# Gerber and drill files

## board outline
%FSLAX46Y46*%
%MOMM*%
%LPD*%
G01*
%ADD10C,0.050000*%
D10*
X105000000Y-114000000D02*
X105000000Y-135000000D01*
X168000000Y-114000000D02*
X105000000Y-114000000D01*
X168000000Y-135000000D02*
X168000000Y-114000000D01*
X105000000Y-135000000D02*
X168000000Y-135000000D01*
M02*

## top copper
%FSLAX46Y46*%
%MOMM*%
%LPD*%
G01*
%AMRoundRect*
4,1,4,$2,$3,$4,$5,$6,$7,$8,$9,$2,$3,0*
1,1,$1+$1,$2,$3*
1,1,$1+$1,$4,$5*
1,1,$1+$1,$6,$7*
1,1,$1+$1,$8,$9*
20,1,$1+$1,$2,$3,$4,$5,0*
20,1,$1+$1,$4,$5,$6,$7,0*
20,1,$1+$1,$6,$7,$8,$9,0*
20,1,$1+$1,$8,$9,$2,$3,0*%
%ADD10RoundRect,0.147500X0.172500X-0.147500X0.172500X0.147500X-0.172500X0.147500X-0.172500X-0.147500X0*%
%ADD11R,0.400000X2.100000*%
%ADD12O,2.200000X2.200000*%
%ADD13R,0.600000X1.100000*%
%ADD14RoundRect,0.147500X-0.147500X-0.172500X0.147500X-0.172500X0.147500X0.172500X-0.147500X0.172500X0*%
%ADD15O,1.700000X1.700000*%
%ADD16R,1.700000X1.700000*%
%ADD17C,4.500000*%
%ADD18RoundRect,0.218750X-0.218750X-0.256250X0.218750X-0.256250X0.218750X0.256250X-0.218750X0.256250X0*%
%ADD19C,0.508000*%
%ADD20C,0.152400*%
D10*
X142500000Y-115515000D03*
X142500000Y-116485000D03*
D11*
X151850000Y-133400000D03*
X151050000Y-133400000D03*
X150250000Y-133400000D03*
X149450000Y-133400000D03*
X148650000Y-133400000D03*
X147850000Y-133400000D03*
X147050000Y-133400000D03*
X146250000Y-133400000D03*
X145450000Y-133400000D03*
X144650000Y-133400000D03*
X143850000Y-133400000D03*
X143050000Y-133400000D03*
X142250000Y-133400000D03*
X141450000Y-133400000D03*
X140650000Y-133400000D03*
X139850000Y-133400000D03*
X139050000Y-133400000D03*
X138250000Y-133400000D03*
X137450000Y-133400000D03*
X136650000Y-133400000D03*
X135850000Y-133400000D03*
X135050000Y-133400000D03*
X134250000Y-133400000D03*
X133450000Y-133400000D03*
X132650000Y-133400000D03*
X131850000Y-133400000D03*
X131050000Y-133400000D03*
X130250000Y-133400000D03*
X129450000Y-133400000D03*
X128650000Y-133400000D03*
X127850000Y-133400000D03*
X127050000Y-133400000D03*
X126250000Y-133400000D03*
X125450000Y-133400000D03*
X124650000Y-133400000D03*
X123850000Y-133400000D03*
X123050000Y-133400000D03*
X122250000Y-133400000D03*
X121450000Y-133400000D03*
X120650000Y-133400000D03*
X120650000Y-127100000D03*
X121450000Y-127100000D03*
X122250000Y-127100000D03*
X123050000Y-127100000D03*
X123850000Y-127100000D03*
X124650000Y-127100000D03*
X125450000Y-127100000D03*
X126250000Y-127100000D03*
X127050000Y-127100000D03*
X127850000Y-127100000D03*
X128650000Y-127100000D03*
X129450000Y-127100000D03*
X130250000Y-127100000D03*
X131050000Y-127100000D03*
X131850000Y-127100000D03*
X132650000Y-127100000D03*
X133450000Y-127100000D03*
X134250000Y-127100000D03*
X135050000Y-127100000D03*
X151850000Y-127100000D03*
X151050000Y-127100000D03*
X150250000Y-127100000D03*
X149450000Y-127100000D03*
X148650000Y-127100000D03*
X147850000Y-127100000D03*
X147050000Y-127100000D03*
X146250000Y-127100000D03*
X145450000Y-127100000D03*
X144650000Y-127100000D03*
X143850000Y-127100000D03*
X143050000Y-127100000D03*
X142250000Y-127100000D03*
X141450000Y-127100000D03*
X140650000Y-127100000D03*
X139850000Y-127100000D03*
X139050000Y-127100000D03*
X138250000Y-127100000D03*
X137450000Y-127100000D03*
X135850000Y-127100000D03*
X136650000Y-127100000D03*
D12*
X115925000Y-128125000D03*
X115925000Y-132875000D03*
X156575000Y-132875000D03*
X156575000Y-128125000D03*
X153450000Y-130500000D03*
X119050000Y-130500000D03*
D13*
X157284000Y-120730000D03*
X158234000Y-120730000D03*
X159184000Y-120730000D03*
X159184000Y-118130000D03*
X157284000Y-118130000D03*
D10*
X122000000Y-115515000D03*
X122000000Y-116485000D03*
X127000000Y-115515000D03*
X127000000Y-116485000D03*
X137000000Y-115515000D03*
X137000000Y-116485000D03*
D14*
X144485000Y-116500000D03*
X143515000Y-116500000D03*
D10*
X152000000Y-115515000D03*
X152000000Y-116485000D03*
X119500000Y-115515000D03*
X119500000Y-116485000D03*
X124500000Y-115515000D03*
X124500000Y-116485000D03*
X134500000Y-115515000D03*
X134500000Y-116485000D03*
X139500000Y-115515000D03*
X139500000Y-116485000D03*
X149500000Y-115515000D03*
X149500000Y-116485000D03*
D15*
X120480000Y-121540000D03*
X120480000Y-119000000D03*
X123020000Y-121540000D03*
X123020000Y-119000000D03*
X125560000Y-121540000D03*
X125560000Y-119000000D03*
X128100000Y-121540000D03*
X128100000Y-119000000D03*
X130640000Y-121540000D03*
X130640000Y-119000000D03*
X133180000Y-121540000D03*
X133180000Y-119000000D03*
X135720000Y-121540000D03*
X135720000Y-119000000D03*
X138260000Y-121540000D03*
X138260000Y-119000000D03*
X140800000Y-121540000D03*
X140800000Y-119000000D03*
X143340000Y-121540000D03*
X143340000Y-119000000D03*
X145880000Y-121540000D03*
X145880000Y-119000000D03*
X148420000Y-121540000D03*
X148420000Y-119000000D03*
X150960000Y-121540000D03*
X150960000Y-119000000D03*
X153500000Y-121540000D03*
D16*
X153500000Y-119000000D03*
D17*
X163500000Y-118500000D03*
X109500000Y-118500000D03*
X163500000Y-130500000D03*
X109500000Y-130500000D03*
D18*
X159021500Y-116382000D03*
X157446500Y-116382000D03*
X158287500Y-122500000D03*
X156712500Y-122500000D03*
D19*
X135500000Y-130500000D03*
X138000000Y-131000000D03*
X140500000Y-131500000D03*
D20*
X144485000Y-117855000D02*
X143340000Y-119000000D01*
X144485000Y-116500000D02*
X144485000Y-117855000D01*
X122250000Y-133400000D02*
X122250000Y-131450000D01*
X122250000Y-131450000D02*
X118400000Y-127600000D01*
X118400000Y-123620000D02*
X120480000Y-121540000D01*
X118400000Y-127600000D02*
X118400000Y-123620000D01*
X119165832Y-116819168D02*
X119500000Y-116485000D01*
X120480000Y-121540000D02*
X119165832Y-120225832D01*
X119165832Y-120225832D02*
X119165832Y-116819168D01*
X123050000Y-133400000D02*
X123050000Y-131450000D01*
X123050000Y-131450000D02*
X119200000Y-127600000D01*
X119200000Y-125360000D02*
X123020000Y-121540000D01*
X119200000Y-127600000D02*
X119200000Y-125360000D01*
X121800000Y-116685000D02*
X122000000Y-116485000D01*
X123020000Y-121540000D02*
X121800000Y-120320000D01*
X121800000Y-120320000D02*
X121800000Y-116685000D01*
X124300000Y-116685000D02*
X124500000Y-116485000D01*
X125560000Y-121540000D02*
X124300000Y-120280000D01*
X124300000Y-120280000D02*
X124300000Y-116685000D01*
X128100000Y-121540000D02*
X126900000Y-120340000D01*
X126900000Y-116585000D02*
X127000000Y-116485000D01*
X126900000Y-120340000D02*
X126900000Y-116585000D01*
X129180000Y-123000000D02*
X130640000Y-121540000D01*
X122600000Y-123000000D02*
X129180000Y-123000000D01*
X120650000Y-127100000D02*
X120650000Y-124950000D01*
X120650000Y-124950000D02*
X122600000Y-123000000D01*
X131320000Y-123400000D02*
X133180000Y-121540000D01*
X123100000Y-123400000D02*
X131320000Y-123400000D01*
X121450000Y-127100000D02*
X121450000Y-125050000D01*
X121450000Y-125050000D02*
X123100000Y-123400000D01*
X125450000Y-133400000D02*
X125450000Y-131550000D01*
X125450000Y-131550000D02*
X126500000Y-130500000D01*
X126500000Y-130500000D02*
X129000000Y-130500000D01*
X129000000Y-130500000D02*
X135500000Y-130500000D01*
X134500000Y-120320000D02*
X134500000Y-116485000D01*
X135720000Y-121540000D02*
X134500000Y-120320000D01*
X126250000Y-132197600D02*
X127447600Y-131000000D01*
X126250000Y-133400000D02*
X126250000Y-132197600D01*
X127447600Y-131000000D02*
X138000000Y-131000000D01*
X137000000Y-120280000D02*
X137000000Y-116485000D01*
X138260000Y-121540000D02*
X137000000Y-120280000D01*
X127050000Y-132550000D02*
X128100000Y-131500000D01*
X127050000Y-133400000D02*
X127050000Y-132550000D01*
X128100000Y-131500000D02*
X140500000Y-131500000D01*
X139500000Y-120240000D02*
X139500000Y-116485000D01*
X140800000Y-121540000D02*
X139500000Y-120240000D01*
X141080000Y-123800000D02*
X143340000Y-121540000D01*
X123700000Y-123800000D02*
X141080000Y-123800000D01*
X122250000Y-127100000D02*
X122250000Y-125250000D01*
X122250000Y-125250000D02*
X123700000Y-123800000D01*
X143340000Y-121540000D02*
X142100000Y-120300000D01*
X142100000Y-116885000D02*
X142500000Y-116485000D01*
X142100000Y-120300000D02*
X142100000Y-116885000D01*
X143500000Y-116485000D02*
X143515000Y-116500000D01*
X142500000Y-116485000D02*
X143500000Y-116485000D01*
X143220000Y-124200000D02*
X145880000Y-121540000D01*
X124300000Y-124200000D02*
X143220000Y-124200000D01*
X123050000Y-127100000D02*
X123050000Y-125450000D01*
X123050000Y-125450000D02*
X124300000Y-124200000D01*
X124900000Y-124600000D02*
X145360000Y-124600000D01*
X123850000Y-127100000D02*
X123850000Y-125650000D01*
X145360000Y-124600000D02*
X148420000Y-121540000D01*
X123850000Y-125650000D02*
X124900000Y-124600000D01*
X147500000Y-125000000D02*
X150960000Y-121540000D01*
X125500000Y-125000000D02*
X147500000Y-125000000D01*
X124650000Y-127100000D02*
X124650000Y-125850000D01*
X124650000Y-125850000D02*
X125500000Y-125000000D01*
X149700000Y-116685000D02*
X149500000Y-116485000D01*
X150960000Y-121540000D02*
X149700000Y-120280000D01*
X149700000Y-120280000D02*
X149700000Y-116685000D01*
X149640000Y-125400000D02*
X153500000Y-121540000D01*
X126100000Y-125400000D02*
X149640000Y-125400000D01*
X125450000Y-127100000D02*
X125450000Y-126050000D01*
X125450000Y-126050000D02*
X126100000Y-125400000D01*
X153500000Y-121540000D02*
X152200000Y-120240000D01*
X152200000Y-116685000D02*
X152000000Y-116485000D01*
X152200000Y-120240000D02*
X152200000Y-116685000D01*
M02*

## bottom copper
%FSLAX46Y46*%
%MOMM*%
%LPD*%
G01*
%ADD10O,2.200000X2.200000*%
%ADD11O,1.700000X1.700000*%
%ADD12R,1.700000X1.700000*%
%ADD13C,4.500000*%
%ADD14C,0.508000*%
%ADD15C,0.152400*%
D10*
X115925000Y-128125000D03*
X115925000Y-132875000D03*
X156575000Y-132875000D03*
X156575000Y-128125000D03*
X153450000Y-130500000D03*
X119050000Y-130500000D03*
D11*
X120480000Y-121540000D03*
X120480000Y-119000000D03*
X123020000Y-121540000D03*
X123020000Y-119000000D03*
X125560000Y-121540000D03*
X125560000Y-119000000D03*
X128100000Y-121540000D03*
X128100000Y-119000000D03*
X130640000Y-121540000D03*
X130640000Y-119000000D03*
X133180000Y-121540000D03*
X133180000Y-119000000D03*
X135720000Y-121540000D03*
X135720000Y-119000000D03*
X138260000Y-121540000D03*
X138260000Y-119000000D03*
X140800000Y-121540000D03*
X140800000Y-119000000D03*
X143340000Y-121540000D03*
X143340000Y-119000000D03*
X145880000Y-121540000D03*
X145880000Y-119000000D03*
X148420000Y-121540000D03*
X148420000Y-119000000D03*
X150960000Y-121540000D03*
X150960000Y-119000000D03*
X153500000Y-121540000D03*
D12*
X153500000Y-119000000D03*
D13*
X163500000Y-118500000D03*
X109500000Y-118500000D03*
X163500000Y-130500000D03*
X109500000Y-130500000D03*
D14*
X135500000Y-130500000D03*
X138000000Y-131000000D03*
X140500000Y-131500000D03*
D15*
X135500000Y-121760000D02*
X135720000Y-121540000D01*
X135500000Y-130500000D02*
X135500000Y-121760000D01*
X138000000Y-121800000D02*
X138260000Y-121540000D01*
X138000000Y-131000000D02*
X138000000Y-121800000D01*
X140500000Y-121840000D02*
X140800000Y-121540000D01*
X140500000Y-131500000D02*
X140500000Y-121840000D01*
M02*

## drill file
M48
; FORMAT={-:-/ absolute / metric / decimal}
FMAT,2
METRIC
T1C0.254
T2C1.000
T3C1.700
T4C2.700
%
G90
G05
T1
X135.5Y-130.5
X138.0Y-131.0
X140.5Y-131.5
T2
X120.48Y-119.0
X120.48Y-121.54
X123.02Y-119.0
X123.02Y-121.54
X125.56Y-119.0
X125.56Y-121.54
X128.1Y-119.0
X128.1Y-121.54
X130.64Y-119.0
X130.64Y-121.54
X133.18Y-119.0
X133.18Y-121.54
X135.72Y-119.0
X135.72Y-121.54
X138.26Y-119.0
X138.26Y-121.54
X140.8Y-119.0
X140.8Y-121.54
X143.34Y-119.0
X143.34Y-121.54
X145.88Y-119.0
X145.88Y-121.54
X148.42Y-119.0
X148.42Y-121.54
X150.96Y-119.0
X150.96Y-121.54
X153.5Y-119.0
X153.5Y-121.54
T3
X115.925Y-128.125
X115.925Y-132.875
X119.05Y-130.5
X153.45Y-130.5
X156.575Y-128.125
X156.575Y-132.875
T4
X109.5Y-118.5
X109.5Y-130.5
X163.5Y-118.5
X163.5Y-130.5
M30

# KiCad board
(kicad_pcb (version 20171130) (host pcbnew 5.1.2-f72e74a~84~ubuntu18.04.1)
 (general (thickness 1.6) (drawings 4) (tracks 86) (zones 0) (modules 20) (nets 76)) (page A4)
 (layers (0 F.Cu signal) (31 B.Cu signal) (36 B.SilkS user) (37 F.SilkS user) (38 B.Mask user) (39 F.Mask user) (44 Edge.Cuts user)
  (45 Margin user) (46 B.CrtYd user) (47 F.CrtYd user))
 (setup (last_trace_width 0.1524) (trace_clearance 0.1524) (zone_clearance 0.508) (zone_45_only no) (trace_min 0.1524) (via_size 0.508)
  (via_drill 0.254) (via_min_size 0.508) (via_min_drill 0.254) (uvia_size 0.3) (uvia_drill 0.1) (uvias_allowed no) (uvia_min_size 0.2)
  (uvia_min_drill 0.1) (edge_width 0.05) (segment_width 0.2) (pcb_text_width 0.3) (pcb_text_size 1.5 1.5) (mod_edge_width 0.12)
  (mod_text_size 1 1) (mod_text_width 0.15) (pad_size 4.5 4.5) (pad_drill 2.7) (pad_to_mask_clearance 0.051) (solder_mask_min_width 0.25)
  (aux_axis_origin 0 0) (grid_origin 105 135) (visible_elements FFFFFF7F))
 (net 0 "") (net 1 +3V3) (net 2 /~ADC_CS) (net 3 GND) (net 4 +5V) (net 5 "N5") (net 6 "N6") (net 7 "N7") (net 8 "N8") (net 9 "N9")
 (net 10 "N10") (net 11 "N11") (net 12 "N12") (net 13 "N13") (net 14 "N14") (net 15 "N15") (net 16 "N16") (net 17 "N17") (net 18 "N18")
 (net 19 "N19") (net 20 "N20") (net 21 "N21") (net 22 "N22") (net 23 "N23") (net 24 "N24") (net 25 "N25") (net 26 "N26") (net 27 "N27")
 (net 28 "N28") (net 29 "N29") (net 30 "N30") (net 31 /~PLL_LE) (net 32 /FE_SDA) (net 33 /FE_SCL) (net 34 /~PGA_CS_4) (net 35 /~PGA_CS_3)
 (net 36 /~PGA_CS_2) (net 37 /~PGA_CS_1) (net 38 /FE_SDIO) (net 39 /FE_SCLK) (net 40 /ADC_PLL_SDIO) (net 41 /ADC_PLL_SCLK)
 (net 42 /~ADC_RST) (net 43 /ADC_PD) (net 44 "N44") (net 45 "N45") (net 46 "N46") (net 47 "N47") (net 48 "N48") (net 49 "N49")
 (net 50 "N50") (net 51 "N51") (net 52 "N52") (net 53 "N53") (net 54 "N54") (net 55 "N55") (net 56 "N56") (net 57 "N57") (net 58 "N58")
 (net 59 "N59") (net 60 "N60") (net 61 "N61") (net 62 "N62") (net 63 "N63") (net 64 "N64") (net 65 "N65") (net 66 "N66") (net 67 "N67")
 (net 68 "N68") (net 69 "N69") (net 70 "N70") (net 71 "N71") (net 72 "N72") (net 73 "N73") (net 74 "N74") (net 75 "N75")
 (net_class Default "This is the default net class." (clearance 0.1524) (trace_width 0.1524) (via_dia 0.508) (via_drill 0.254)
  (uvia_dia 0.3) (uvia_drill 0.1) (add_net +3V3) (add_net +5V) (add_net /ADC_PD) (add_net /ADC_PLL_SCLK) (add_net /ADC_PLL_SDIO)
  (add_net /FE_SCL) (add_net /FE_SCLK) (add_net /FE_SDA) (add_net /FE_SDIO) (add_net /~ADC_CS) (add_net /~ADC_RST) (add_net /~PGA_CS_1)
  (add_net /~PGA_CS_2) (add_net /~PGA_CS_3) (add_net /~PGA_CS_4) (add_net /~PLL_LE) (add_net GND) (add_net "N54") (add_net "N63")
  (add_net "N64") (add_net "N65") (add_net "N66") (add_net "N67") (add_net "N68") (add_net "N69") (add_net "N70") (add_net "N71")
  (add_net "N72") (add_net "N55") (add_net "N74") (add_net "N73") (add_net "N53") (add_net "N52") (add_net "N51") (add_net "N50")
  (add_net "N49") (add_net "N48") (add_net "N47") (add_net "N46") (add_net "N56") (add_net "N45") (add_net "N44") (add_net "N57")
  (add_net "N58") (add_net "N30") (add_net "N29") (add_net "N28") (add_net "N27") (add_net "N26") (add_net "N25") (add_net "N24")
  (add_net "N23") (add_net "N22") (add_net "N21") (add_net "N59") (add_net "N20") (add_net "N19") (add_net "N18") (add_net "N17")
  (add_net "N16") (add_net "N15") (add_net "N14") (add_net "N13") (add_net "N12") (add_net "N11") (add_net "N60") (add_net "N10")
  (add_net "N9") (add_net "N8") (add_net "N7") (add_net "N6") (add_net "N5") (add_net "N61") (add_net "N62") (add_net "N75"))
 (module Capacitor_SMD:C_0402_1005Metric (layer F.Cu) (at 142.5 116 90)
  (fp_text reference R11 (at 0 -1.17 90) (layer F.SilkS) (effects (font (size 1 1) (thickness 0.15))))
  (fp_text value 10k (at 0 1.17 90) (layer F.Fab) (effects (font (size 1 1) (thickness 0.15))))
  (pad 2 smd roundrect (at 0.485 0 90) (size 0.59 0.64) (layers F.Cu F.Paste F.Mask) (roundrect_rratio 0.25) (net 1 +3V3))
  (pad 1 smd roundrect (at -0.485 0 90) (size 0.59 0.64) (layers F.Cu F.Paste F.Mask) (roundrect_rratio 0.25) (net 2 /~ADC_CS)))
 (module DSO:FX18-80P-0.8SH (layer F.Cu) (at 136.25 130.5 180)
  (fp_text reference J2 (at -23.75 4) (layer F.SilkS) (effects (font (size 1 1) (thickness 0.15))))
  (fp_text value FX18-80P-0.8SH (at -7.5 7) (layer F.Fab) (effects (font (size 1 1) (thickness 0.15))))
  (pad 80 smd rect (at -15.6 -2.9 180) (size 0.4 2.1) (layers F.Cu F.Paste F.Mask) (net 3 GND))
  (pad 79 smd rect (at -14.8 -2.9 180) (size 0.4 2.1) (layers F.Cu F.Paste F.Mask) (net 3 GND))
  (pad 78 smd rect (at -14 -2.9 180) (size 0.4 2.1) (layers F.Cu F.Paste F.Mask) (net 3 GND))
  (pad 77 smd rect (at -13.2 -2.9 180) (size 0.4 2.1) (layers F.Cu F.Paste F.Mask) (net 3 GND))
  (pad 76 smd rect (at -12.4 -2.9 180) (size 0.4 2.1) (layers F.Cu F.Paste F.Mask) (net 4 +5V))
  (pad 75 smd rect (at -11.6 -2.9 180) (size 0.4 2.1) (layers F.Cu F.Paste F.Mask) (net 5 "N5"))
  (pad 74 smd rect (at -10.8 -2.9 180) (size 0.4 2.1) (layers F.Cu F.Paste F.Mask) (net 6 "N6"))
  (pad 73 smd rect (at -10 -2.9 180) (size 0.4 2.1) (layers F.Cu F.Paste F.Mask) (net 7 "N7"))
  (pad 72 smd rect (at -9.2 -2.9 180) (size 0.4 2.1) (layers F.Cu F.Paste F.Mask) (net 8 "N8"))
  (pad 71 smd rect (at -8.4 -2.9 180) (size 0.4 2.1) (layers F.Cu F.Paste F.Mask) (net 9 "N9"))
  (pad 70 smd rect (at -7.6 -2.9 180) (size 0.4 2.1) (layers F.Cu F.Paste F.Mask) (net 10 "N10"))
  (pad 69 smd rect (at -6.8 -2.9 180) (size 0.4 2.1) (layers F.Cu F.Paste F.Mask) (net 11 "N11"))
  (pad 68 smd rect (at -6 -2.9 180) (size 0.4 2.1) (layers F.Cu F.Paste F.Mask) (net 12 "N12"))
  (pad 67 smd rect (at -5.2 -2.9 180) (size 0.4 2.1) (layers F.Cu F.Paste F.Mask) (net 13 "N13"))
  (pad 66 smd rect (at -4.4 -2.9 180) (size 0.4 2.1) (layers F.Cu F.Paste F.Mask) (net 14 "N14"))
  (pad 65 smd rect (at -3.6 -2.9 180) (size 0.4 2.1) (layers F.Cu F.Paste F.Mask) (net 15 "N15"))
  (pad 64 smd rect (at -2.8 -2.9 180) (size 0.4 2.1) (layers F.Cu F.Paste F.Mask) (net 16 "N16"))
  (pad 63 smd rect (at -2 -2.9 180) (size 0.4 2.1) (layers F.Cu F.Paste F.Mask) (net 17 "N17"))
  (pad 62 smd rect (at -1.2 -2.9 180) (size 0.4 2.1) (layers F.Cu F.Paste F.Mask) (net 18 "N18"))
  (pad 61 smd rect (at -0.4 -2.9 180) (size 0.4 2.1) (layers F.Cu F.Paste F.Mask) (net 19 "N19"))
  (pad 60 smd rect (at 0.4 -2.9 180) (size 0.4 2.1) (layers F.Cu F.Paste F.Mask) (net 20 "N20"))
  (pad 59 smd rect (at 1.2 -2.9 180) (size 0.4 2.1) (layers F.Cu F.Paste F.Mask) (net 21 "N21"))
  (pad 58 smd rect (at 2 -2.9 180) (size 0.4 2.1) (layers F.Cu F.Paste F.Mask) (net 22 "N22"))
  (pad 57 smd rect (at 2.8 -2.9 180) (size 0.4 2.1) (layers F.Cu F.Paste F.Mask) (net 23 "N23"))
  (pad 56 smd rect (at 3.6 -2.9 180) (size 0.4 2.1) (layers F.Cu F.Paste F.Mask) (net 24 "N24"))
  (pad 55 smd rect (at 4.4 -2.9 180) (size 0.4 2.1) (layers F.Cu F.Paste F.Mask) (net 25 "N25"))
  (pad 54 smd rect (at 5.2 -2.9 180) (size 0.4 2.1) (layers F.Cu F.Paste F.Mask) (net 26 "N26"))
  (pad 53 smd rect (at 6 -2.9 180) (size 0.4 2.1) (layers F.Cu F.Paste F.Mask) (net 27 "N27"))
  (pad 52 smd rect (at 6.8 -2.9 180) (size 0.4 2.1) (layers F.Cu F.Paste F.Mask) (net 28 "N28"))
  (pad 51 smd rect (at 7.6 -2.9 180) (size 0.4 2.1) (layers F.Cu F.Paste F.Mask) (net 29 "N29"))
  (pad 50 smd rect (at 8.4 -2.9 180) (size 0.4 2.1) (layers F.Cu F.Paste F.Mask) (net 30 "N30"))
  (pad 49 smd rect (at 9.2 -2.9 180) (size 0.4 2.1) (layers F.Cu F.Paste F.Mask) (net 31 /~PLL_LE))
  (pad 48 smd rect (at 10 -2.9 180) (size 0.4 2.1) (layers F.Cu F.Paste F.Mask) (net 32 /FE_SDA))
  (pad 47 smd rect (at 10.8 -2.9 180) (size 0.4 2.1) (layers F.Cu F.Paste F.Mask) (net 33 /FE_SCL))
  (pad 46 smd rect (at 11.6 -2.9 180) (size 0.4 2.1) (layers F.Cu F.Paste F.Mask) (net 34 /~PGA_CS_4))
  (pad 45 smd rect (at 12.4 -2.9 180) (size 0.4 2.1) (layers F.Cu F.Paste F.Mask) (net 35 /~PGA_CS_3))
  (pad 44 smd rect (at 13.2 -2.9 180) (size 0.4 2.1) (layers F.Cu F.Paste F.Mask) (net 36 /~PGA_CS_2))
  (pad 43 smd rect (at 14 -2.9 180) (size 0.4 2.1) (layers F.Cu F.Paste F.Mask) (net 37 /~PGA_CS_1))
  (pad 42 smd rect (at 14.8 -2.9 180) (size 0.4 2.1) (layers F.Cu F.Paste F.Mask) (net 3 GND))
  (pad 41 smd rect (at 15.6 -2.9 180) (size 0.4 2.1) (layers F.Cu F.Paste F.Mask) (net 3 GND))
  (pad 40 smd rect (at 15.6 3.4 180) (size 0.4 2.1) (layers F.Cu F.Paste F.Mask) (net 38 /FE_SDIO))
  (pad 39 smd rect (at 14.8 3.4 180) (size 0.4 2.1) (layers F.Cu F.Paste F.Mask) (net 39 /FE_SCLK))
  (pad 38 smd rect (at 14 3.4 180) (size 0.4 2.1) (layers F.Cu F.Paste F.Mask) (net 2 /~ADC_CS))
  (pad 37 smd rect (at 13.2 3.4 180) (size 0.4 2.1) (layers F.Cu F.Paste F.Mask) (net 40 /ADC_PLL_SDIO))
  (pad 36 smd rect (at 12.4 3.4 180) (size 0.4 2.1) (layers F.Cu F.Paste F.Mask) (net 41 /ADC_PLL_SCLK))
  (pad 35 smd rect (at 11.6 3.4 180) (size 0.4 2.1) (layers F.Cu F.Paste F.Mask) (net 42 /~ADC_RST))
  (pad 34 smd rect (at 10.8 3.4 180) (size 0.4 2.1) (layers F.Cu F.Paste F.Mask) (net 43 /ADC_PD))
  (pad 33 smd rect (at 10 3.4 180) (size 0.4 2.1) (layers F.Cu F.Paste F.Mask) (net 3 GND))
  (pad 32 smd rect (at 9.2 3.4 180) (size 0.4 2.1) (layers F.Cu F.Paste F.Mask) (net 3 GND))
  (pad 31 smd rect (at 8.4 3.4 180) (size 0.4 2.1) (layers F.Cu F.Paste F.Mask) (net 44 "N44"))
  (pad 30 smd rect (at 7.6 3.4 180) (size 0.4 2.1) (layers F.Cu F.Paste F.Mask) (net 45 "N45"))
  (pad 29 smd rect (at 6.8 3.4 180) (size 0.4 2.1) (layers F.Cu F.Paste F.Mask) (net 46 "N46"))
  (pad 28 smd rect (at 6 3.4 180) (size 0.4 2.1) (layers F.Cu F.Paste F.Mask) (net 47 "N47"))
  (pad 27 smd rect (at 5.2 3.4 180) (size 0.4 2.1) (layers F.Cu F.Paste F.Mask) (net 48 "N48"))
  (pad 26 smd rect (at 4.4 3.4 180) (size 0.4 2.1) (layers F.Cu F.Paste F.Mask) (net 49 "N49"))
  (pad 25 smd rect (at 3.6 3.4 180) (size 0.4 2.1) (layers F.Cu F.Paste F.Mask) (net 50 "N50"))
  (pad 24 smd rect (at 2.8 3.4 180) (size 0.4 2.1) (layers F.Cu F.Paste F.Mask) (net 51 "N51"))
  (pad 23 smd rect (at 2 3.4 180) (size 0.4 2.1) (layers F.Cu F.Paste F.Mask) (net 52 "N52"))
  (pad 22 smd rect (at 1.2 3.4 180) (size 0.4 2.1) (layers F.Cu F.Paste F.Mask) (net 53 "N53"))
  (pad 1 smd rect (at -15.6 3.4 180) (size 0.4 2.1) (layers F.Cu F.Paste F.Mask) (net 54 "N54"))
  (pad 2 smd rect (at -14.8 3.4 180) (size 0.4 2.1) (layers F.Cu F.Paste F.Mask) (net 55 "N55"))
  (pad 3 smd rect (at -14 3.4 180) (size 0.4 2.1) (layers F.Cu F.Paste F.Mask) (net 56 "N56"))
  (pad 4 smd rect (at -13.2 3.4 180) (size 0.4 2.1) (layers F.Cu F.Paste F.Mask) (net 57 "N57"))
  (pad 5 smd rect (at -12.4 3.4 180) (size 0.4 2.1) (layers F.Cu F.Paste F.Mask) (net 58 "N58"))
  (pad 6 smd rect (at -11.6 3.4 180) (size 0.4 2.1) (layers F.Cu F.Paste F.Mask) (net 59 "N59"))
  (pad 7 smd rect (at -10.8 3.4 180) (size 0.4 2.1) (layers F.Cu F.Paste F.Mask) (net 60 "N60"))
  (pad 8 smd rect (at -10 3.4 180) (size 0.4 2.1) (layers F.Cu F.Paste F.Mask) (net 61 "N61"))
  (pad 9 smd rect (at -9.2 3.4 180) (size 0.4 2.1) (layers F.Cu F.Paste F.Mask) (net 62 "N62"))
  (pad 10 smd rect (at -8.4 3.4 180) (size 0.4 2.1) (layers F.Cu F.Paste F.Mask) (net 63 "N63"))
  (pad 11 smd rect (at -7.6 3.4 180) (size 0.4 2.1) (layers F.Cu F.Paste F.Mask) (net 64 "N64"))
  (pad 12 smd rect (at -6.8 3.4 180) (size 0.4 2.1) (layers F.Cu F.Paste F.Mask) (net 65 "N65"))
  (pad 13 smd rect (at -6 3.4 180) (size 0.4 2.1) (layers F.Cu F.Paste F.Mask) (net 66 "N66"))
  (pad 14 smd rect (at -5.2 3.4 180) (size 0.4 2.1) (layers F.Cu F.Paste F.Mask) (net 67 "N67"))
  (pad 15 smd rect (at -4.4 3.4 180) (size 0.4 2.1) (layers F.Cu F.Paste F.Mask) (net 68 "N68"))
  (pad 16 smd rect (at -3.6 3.4 180) (size 0.4 2.1) (layers F.Cu F.Paste F.Mask) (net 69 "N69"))
  (pad 17 smd rect (at -2.8 3.4 180) (size 0.4 2.1) (layers F.Cu F.Paste F.Mask) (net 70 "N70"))
  (pad 18 smd rect (at -2 3.4 180) (size 0.4 2.1) (layers F.Cu F.Paste F.Mask) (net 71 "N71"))
  (pad 19 smd rect (at -1.2 3.4 180) (size 0.4 2.1) (layers F.Cu F.Paste F.Mask) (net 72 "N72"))
  (pad 21 smd rect (at 0.4 3.4 180) (size 0.4 2.1) (layers F.Cu F.Paste F.Mask) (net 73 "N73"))
  (pad 20 smd rect (at -0.4 3.4 180) (size 0.4 2.1) (layers F.Cu F.Paste F.Mask) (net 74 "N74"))
  (pad SHLD thru_hole oval (at 20.325 2.375 180) (size 2.2 2.2) (drill 1.7) (layers *.Cu *.Mask) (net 3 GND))
  (pad SHLD thru_hole oval (at 20.325 -2.375 180) (size 2.2 2.2) (drill 1.7) (layers *.Cu *.Mask) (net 3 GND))
  (pad SHLD thru_hole oval (at -20.325 -2.375 180) (size 2.2 2.2) (drill 1.7) (layers *.Cu *.Mask) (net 3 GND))
  (pad SHLD thru_hole oval (at -20.325 2.375 180) (size 2.2 2.2) (drill 1.7) (layers *.Cu *.Mask) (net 3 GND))
  (pad SHLD thru_hole oval (at -17.2 0 180) (size 2.2 2.2) (drill 1.7) (layers *.Cu *.Mask) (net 3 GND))
  (pad SHLD thru_hole oval (at 17.2 0 180) (size 2.2 2.2) (drill 1.7) (layers *.Cu *.Mask) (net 3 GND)))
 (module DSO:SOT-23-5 (layer F.Cu) (at 158.234 119.43 90) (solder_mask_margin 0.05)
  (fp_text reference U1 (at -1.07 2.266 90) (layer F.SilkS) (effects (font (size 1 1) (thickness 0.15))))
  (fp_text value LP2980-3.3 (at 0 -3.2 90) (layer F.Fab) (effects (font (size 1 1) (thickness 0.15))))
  (pad 1 smd rect (at -1.3 -0.95 90) (size 1.1 0.6) (layers F.Cu F.Paste F.Mask) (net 4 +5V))
  (pad 2 smd rect (at -1.3 0 90) (size 1.1 0.6) (layers F.Cu F.Paste F.Mask) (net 3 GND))
  (pad 3 smd rect (at -1.3 0.95 90) (size 1.1 0.6) (layers F.Cu F.Paste F.Mask) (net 4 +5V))
  (pad 4 smd rect (at 1.3 0.95 90) (size 1.1 0.6) (layers F.Cu F.Paste F.Mask) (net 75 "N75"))
  (pad 5 smd rect (at 1.3 -0.95 90) (size 1.1 0.6) (layers F.Cu F.Paste F.Mask) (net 1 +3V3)))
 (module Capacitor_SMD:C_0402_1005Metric (layer F.Cu) (at 122 116 90)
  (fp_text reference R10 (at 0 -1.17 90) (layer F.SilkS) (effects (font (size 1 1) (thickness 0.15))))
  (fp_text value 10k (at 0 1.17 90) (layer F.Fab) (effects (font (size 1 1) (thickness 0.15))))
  (pad 2 smd roundrect (at 0.485 0 90) (size 0.59 0.64) (layers F.Cu F.Paste F.Mask) (roundrect_rratio 0.25) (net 1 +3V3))
  (pad 1 smd roundrect (at -0.485 0 90) (size 0.59 0.64) (layers F.Cu F.Paste F.Mask) (roundrect_rratio 0.25) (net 36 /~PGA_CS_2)))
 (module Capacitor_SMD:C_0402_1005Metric (layer F.Cu) (at 127 116 90)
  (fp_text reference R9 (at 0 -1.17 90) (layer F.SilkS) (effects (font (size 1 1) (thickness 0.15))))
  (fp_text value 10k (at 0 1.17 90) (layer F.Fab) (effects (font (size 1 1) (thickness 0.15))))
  (pad 2 smd roundrect (at 0.485 0 90) (size 0.59 0.64) (layers F.Cu F.Paste F.Mask) (roundrect_rratio 0.25) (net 1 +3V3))
  (pad 1 smd roundrect (at -0.485 0 90) (size 0.59 0.64) (layers F.Cu F.Paste F.Mask) (roundrect_rratio 0.25) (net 34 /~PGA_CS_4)))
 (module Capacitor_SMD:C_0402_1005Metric (layer F.Cu) (at 137 116 90)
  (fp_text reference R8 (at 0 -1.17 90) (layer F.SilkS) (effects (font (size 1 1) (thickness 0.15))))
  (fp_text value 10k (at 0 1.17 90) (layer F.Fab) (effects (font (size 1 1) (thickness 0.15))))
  (pad 2 smd roundrect (at 0.485 0 90) (size 0.59 0.64) (layers F.Cu F.Paste F.Mask) (roundrect_rratio 0.25) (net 1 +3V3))
  (pad 1 smd roundrect (at -0.485 0 90) (size 0.59 0.64) (layers F.Cu F.Paste F.Mask) (roundrect_rratio 0.25) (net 32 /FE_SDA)))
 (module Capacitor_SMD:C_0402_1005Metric (layer F.Cu) (at 144 116.5)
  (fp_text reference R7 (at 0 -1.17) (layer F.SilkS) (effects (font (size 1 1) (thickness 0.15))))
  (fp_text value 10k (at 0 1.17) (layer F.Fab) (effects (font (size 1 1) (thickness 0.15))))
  (pad 2 smd roundrect (at 0.485 0) (size 0.59 0.64) (layers F.Cu F.Paste F.Mask) (roundrect_rratio 0.25) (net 3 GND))
  (pad 1 smd roundrect (at -0.485 0) (size 0.59 0.64) (layers F.Cu F.Paste F.Mask) (roundrect_rratio 0.25) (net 2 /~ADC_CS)))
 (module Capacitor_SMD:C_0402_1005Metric (layer F.Cu) (at 152 116 90)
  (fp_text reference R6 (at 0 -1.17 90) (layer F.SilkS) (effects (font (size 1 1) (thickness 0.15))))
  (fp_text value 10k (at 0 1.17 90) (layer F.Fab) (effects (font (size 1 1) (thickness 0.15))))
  (pad 2 smd roundrect (at 0.485 0 90) (size 0.59 0.64) (layers F.Cu F.Paste F.Mask) (roundrect_rratio 0.25) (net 1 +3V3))
  (pad 1 smd roundrect (at -0.485 0 90) (size 0.59 0.64) (layers F.Cu F.Paste F.Mask) (roundrect_rratio 0.25) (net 43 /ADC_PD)))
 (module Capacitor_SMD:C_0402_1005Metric (layer F.Cu) (at 119.5 116 90)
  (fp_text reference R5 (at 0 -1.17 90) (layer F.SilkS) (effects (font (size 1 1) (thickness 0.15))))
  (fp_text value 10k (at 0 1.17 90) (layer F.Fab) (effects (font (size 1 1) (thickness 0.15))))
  (pad 2 smd roundrect (at 0.485 0 90) (size 0.59 0.64) (layers F.Cu F.Paste F.Mask) (roundrect_rratio 0.25) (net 1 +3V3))
  (pad 1 smd roundrect (at -0.485 0 90) (size 0.59 0.64) (layers F.Cu F.Paste F.Mask) (roundrect_rratio 0.25) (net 37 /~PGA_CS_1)))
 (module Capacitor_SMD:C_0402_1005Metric (layer F.Cu) (at 124.5 116 90)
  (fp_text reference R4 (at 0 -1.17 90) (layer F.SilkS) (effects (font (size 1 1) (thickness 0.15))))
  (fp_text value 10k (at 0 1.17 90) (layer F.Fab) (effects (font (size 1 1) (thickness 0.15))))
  (pad 2 smd roundrect (at 0.485 0 90) (size 0.59 0.64) (layers F.Cu F.Paste F.Mask) (roundrect_rratio 0.25) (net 1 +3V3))
  (pad 1 smd roundrect (at -0.485 0 90) (size 0.59 0.64) (layers F.Cu F.Paste F.Mask) (roundrect_rratio 0.25) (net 35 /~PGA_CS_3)))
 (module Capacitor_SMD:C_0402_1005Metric (layer F.Cu) (at 134.5 116 90)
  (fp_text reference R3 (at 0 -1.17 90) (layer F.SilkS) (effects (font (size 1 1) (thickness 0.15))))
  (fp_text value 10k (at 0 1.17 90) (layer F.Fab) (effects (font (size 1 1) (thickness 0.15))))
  (pad 2 smd roundrect (at 0.485 0 90) (size 0.59 0.64) (layers F.Cu F.Paste F.Mask) (roundrect_rratio 0.25) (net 1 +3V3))
  (pad 1 smd roundrect (at -0.485 0 90) (size 0.59 0.64) (layers F.Cu F.Paste F.Mask) (roundrect_rratio 0.25) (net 33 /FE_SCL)))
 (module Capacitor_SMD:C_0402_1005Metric (layer F.Cu) (at 139.5 116 90)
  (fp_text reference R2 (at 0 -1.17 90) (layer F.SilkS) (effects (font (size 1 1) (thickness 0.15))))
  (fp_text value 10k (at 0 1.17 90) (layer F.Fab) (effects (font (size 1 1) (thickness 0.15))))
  (pad 2 smd roundrect (at 0.485 0 90) (size 0.59 0.64) (layers F.Cu F.Paste F.Mask) (roundrect_rratio 0.25) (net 1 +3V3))
  (pad 1 smd roundrect (at -0.485 0 90) (size 0.59 0.64) (layers F.Cu F.Paste F.Mask) (roundrect_rratio 0.25) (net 31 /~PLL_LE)))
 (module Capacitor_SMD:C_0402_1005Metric (layer F.Cu) (at 149.5 116 90)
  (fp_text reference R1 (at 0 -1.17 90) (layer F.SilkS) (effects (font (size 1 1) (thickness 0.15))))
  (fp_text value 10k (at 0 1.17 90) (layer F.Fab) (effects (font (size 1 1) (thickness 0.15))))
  (pad 2 smd roundrect (at 0.485 0 90) (size 0.59 0.64) (layers F.Cu F.Paste F.Mask) (roundrect_rratio 0.25) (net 1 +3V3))
  (pad 1 smd roundrect (at -0.485 0 90) (size 0.59 0.64) (layers F.Cu F.Paste F.Mask) (roundrect_rratio 0.25) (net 42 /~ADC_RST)))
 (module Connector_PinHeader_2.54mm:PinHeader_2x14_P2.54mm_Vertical (layer F.Cu) (at 153.5 119 270)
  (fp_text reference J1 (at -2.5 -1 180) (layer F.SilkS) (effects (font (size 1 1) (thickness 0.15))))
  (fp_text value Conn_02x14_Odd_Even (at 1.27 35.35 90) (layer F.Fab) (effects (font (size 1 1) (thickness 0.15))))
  (pad 28 thru_hole oval (at 2.54 33.02 270) (size 1.7 1.7) (drill 1) (layers *.Cu *.Mask) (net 37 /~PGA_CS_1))
  (pad 27 thru_hole oval (at 0 33.02 270) (size 1.7 1.7) (drill 1) (layers *.Cu *.Mask) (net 3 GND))
  (pad 26 thru_hole oval (at 2.54 30.48 270) (size 1.7 1.7) (drill 1) (layers *.Cu *.Mask) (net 36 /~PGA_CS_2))
  (pad 25 thru_hole oval (at 0 30.48 270) (size 1.7 1.7) (drill 1) (layers *.Cu *.Mask) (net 3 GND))
  (pad 24 thru_hole oval (at 2.54 27.94 270) (size 1.7 1.7) (drill 1) (layers *.Cu *.Mask) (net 35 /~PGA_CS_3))
  (pad 23 thru_hole oval (at 0 27.94 270) (size 1.7 1.7) (drill 1) (layers *.Cu *.Mask) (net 3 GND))
  (pad 22 thru_hole oval (at 2.54 25.4 270) (size 1.7 1.7) (drill 1) (layers *.Cu *.Mask) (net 34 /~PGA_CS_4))
  (pad 21 thru_hole oval (at 0 25.4 270) (size 1.7 1.7) (drill 1) (layers *.Cu *.Mask) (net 3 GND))
  (pad 20 thru_hole oval (at 2.54 22.86 270) (size 1.7 1.7) (drill 1) (layers *.Cu *.Mask) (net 38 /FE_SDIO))
  (pad 19 thru_hole oval (at 0 22.86 270) (size 1.7 1.7) (drill 1) (layers *.Cu *.Mask) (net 3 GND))
  (pad 18 thru_hole oval (at 2.54 20.32 270) (size 1.7 1.7) (drill 1) (layers *.Cu *.Mask) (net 39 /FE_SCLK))
  (pad 17 thru_hole oval (at 0 20.32 270) (size 1.7 1.7) (drill 1) (layers *.Cu *.Mask) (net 3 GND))
  (pad 16 thru_hole oval (at 2.54 17.78 270) (size 1.7 1.7) (drill 1) (layers *.Cu *.Mask) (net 33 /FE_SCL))
  (pad 15 thru_hole oval (at 0 17.78 270) (size 1.7 1.7) (drill 1) (layers *.Cu *.Mask) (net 3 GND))
  (pad 14 thru_hole oval (at 2.54 15.24 270) (size 1.7 1.7) (drill 1) (layers *.Cu *.Mask) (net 32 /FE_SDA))
  (pad 13 thru_hole oval (at 0 15.24 270) (size 1.7 1.7) (drill 1) (layers *.Cu *.Mask) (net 3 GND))
  (pad 12 thru_hole oval (at 2.54 12.7 270) (size 1.7 1.7) (drill 1) (layers *.Cu *.Mask) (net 31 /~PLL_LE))
  (pad 11 thru_hole oval (at 0 12.7 270) (size 1.7 1.7) (drill 1) (layers *.Cu *.Mask) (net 3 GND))
  (pad 10 thru_hole oval (at 2.54 10.16 270) (size 1.7 1.7) (drill 1) (layers *.Cu *.Mask) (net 2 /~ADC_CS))
  (pad 9 thru_hole oval (at 0 10.16 270) (size 1.7 1.7) (drill 1) (layers *.Cu *.Mask) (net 3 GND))
  (pad 8 thru_hole oval (at 2.54 7.62 270) (size 1.7 1.7) (drill 1) (layers *.Cu *.Mask) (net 40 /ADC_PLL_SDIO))
  (pad 7 thru_hole oval (at 0 7.62 270) (size 1.7 1.7) (drill 1) (layers *.Cu *.Mask) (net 3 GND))
  (pad 6 thru_hole oval (at 2.54 5.08 270) (size 1.7 1.7) (drill 1) (layers *.Cu *.Mask) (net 41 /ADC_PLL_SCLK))
  (pad 5 thru_hole oval (at 0 5.08 270) (size 1.7 1.7) (drill 1) (layers *.Cu *.Mask) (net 3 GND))
  (pad 4 thru_hole oval (at 2.54 2.54 270) (size 1.7 1.7) (drill 1) (layers *.Cu *.Mask) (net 42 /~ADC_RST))
  (pad 3 thru_hole oval (at 0 2.54 270) (size 1.7 1.7) (drill 1) (layers *.Cu *.Mask) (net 3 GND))
  (pad 2 thru_hole oval (at 2.54 0 270) (size 1.7 1.7) (drill 1) (layers *.Cu *.Mask) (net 43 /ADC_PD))
  (pad 1 thru_hole rect (at 0 0 270) (size 1.7 1.7) (drill 1) (layers *.Cu *.Mask) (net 3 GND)))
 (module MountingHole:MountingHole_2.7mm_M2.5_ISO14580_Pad (layer F.Cu) (at 163.5 118.5)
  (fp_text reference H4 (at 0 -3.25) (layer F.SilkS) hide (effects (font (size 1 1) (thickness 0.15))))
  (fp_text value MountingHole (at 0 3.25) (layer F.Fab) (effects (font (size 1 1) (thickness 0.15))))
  (pad 1 thru_hole circle (at 0 0) (size 4.5 4.5) (drill 2.7) (layers *.Cu *.Mask) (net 3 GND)))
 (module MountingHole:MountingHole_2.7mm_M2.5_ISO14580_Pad (layer F.Cu) (at 109.5 118.5)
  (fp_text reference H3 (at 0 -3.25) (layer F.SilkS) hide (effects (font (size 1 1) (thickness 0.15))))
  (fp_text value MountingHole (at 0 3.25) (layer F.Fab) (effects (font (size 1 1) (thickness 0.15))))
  (pad 1 thru_hole circle (at 0 0) (size 4.5 4.5) (drill 2.7) (layers *.Cu *.Mask) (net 3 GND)))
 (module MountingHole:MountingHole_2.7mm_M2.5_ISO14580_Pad (layer F.Cu) (at 163.5 130.5)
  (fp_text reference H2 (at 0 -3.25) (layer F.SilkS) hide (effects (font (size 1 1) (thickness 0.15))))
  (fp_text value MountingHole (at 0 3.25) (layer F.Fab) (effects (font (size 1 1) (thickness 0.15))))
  (pad 1 thru_hole circle (at 0 0) (size 4.5 4.5) (drill 2.7) (layers *.Cu *.Mask) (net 3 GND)))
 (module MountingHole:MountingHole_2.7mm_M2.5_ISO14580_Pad (layer F.Cu) (at 109.5 130.5)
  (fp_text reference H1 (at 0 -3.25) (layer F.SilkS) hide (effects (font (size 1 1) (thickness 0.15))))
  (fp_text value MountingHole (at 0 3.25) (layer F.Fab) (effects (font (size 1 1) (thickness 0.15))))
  (pad 1 thru_hole circle (at 0 0) (size 4.5 4.5) (drill 2.7) (layers *.Cu *.Mask) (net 3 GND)))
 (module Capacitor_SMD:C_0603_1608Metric (layer F.Cu) (at 158.234 116.382)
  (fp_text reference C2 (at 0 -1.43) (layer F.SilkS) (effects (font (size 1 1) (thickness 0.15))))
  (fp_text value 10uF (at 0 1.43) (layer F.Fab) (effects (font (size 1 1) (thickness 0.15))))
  (pad 2 smd roundrect (at 0.7875 0) (size 0.875 0.95) (layers F.Cu F.Paste F.Mask) (roundrect_rratio 0.25) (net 3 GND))
  (pad 1 smd roundrect (at -0.7875 0) (size 0.875 0.95) (layers F.Cu F.Paste F.Mask) (roundrect_rratio 0.25) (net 1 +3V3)))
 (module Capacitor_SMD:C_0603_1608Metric (layer F.Cu) (at 157.5 122.5)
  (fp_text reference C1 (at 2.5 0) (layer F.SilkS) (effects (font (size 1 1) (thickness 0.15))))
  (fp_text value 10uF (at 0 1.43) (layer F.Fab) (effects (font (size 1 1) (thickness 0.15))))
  (pad 2 smd roundrect (at 0.7875 0) (size 0.875 0.95) (layers F.Cu F.Paste F.Mask) (roundrect_rratio 0.25) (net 3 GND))
  (pad 1 smd roundrect (at -0.7875 0) (size 0.875 0.95) (layers F.Cu F.Paste F.Mask) (roundrect_rratio 0.25) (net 4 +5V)))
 (gr_line (start 105 114) (end 105 135) (layer Edge.Cuts) (width 0.05))
 (gr_line (start 168 114) (end 105 114) (layer Edge.Cuts) (width 0.05))
 (gr_line (start 168 135) (end 168 114) (layer Edge.Cuts) (width 0.05))
 (gr_line (start 105 135) (end 168 135) (layer Edge.Cuts) (width 0.05))
 (segment (start 144.485 117.855) (end 143.34 119) (width 0.1524) (layer F.Cu) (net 3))
 (segment (start 144.485 116.5) (end 144.485 117.855) (width 0.1524) (layer F.Cu) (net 3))
 (segment (start 122.25 133.4) (end 122.25 131.45) (width 0.1524) (layer F.Cu) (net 37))
 (segment (start 122.25 131.45) (end 118.4 127.6) (width 0.1524) (layer F.Cu) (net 37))
 (segment (start 118.4 123.62) (end 120.48 121.54) (width 0.1524) (layer F.Cu) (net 37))
 (segment (start 118.4 127.6) (end 118.4 123.62) (width 0.1524) (layer F.Cu) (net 37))
 (segment (start 119.165832 116.819168) (end 119.5 116.485) (width 0.1524) (layer F.Cu) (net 37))
 (segment (start 120.48 121.54) (end 119.165832 120.225832) (width 0.1524) (layer F.Cu) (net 37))
 (segment (start 119.165832 120.225832) (end 119.165832 116.819168) (width 0.1524) (layer F.Cu) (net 37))
 (segment (start 123.05 133.4) (end 123.05 131.45) (width 0.1524) (layer F.Cu) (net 36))
 (segment (start 123.05 131.45) (end 119.2 127.6) (width 0.1524) (layer F.Cu) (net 36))
 (segment (start 119.2 125.36) (end 123.02 121.54) (width 0.1524) (layer F.Cu) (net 36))
 (segment (start 119.2 127.6) (end 119.2 125.36) (width 0.1524) (layer F.Cu) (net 36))
 (segment (start 121.8 116.685) (end 122 116.485) (width 0.1524) (layer F.Cu) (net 36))
 (segment (start 123.02 121.54) (end 121.8 120.32) (width 0.1524) (layer F.Cu) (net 36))
 (segment (start 121.8 120.32) (end 121.8 116.685) (width 0.1524) (layer F.Cu) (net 36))
 (segment (start 124.3 116.685) (end 124.5 116.485) (width 0.1524) (layer F.Cu) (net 35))
 (segment (start 125.56 121.54) (end 124.3 120.28) (width 0.1524) (layer F.Cu) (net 35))
 (segment (start 124.3 120.28) (end 124.3 116.685) (width 0.1524) (layer F.Cu) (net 35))
 (segment (start 128.1 121.54) (end 126.9 120.34) (width 0.1524) (layer F.Cu) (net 34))
 (segment (start 126.9 116.585) (end 127 116.485) (width 0.1524) (layer F.Cu) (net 34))
 (segment (start 126.9 120.34) (end 126.9 116.585) (width 0.1524) (layer F.Cu) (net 34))
 (segment (start 129.18 123) (end 130.64 121.54) (width 0.1524) (layer F.Cu) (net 38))
 (segment (start 122.6 123) (end 129.18 123) (width 0.1524) (layer F.Cu) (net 38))
 (segment (start 120.65 127.1) (end 120.65 124.95) (width 0.1524) (layer F.Cu) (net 38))
 (segment (start 120.65 124.95) (end 122.6 123) (width 0.1524) (layer F.Cu) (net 38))
 (segment (start 131.32 123.4) (end 133.18 121.54) (width 0.1524) (layer F.Cu) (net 39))
 (segment (start 123.1 123.4) (end 131.32 123.4) (width 0.1524) (layer F.Cu) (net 39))
 (segment (start 121.45 127.1) (end 121.45 125.05) (width 0.1524) (layer F.Cu) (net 39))
 (segment (start 121.45 125.05) (end 123.1 123.4) (width 0.1524) (layer F.Cu) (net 39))
 (segment (start 125.45 133.4) (end 125.45 131.55) (width 0.1524) (layer F.Cu) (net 33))
 (segment (start 125.45 131.55) (end 126.5 130.5) (width 0.1524) (layer F.Cu) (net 33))
 (segment (start 126.5 130.5) (end 129 130.5) (width 0.1524) (layer F.Cu) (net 33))
 (segment (start 129 130.5) (end 135.5 130.5) (width 0.1524) (layer F.Cu) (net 33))
 (via (at 135.5 130.5) (size 0.508) (drill 0.254) (layers F.Cu B.Cu) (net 33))
 (segment (start 135.5 121.76) (end 135.72 121.54) (width 0.1524) (layer B.Cu) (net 33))
 (segment (start 135.5 130.5) (end 135.5 121.76) (width 0.1524) (layer B.Cu) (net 33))
 (segment (start 134.5 120.32) (end 134.5 116.485) (width 0.1524) (layer F.Cu) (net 33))
 (segment (start 135.72 121.54) (end 134.5 120.32) (width 0.1524) (layer F.Cu) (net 33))
 (segment (start 126.25 132.1976) (end 127.4476 131) (width 0.1524) (layer F.Cu) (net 32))
 (segment (start 126.25 133.4) (end 126.25 132.1976) (width 0.1524) (layer F.Cu) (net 32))
 (via (at 138 131) (size 0.508) (drill 0.254) (layers F.Cu B.Cu) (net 32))
 (segment (start 127.4476 131) (end 138 131) (width 0.1524) (layer F.Cu) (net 32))
 (segment (start 138 121.8) (end 138.26 121.54) (width 0.1524) (layer B.Cu) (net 32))
 (segment (start 138 131) (end 138 121.8) (width 0.1524) (layer B.Cu) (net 32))
 (segment (start 137 120.28) (end 137 116.485) (width 0.1524) (layer F.Cu) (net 32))
 (segment (start 138.26 121.54) (end 137 120.28) (width 0.1524) (layer F.Cu) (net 32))
 (segment (start 127.05 132.55) (end 128.1 131.5) (width 0.1524) (layer F.Cu) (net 31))
 (segment (start 127.05 133.4) (end 127.05 132.55) (width 0.1524) (layer F.Cu) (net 31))
 (via (at 140.5 131.5) (size 0.508) (drill 0.254) (layers F.Cu B.Cu) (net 31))
 (segment (start 128.1 131.5) (end 140.5 131.5) (width 0.1524) (layer F.Cu) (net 31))
 (segment (start 140.5 121.84) (end 140.8 121.54) (width 0.1524) (layer B.Cu) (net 31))
 (segment (start 140.5 131.5) (end 140.5 121.84) (width 0.1524) (layer B.Cu) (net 31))
 (segment (start 139.5 120.24) (end 139.5 116.485) (width 0.1524) (layer F.Cu) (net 31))
 (segment (start 140.8 121.54) (end 139.5 120.24) (width 0.1524) (layer F.Cu) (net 31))
 (segment (start 141.08 123.8) (end 143.34 121.54) (width 0.1524) (layer F.Cu) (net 2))
 (segment (start 123.7 123.8) (end 141.08 123.8) (width 0.1524) (layer F.Cu) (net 2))
 (segment (start 122.25 127.1) (end 122.25 125.25) (width 0.1524) (layer F.Cu) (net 2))
 (segment (start 122.25 125.25) (end 123.7 123.8) (width 0.1524) (layer F.Cu) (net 2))
 (segment (start 143.34 121.54) (end 142.1 120.3) (width 0.1524) (layer F.Cu) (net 2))
 (segment (start 142.1 116.885) (end 142.5 116.485) (width 0.1524) (layer F.Cu) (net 2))
 (segment (start 142.1 120.3) (end 142.1 116.885) (width 0.1524) (layer F.Cu) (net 2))
 (segment (start 143.5 116.485) (end 143.515 116.5) (width 0.1524) (layer F.Cu) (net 2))
 (segment (start 142.5 116.485) (end 143.5 116.485) (width 0.1524) (layer F.Cu) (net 2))
 (segment (start 143.22 124.2) (end 145.88 121.54) (width 0.1524) (layer F.Cu) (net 40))
 (segment (start 124.3 124.2) (end 143.22 124.2) (width 0.1524) (layer F.Cu) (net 40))
 (segment (start 123.05 127.1) (end 123.05 125.45) (width 0.1524) (layer F.Cu) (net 40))
 (segment (start 123.05 125.45) (end 124.3 124.2) (width 0.1524) (layer F.Cu) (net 40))
 (segment (start 124.9 124.6) (end 145.36 124.6) (width 0.1524) (layer F.Cu) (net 41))
 (segment (start 123.85 127.1) (end 123.85 125.65) (width 0.1524) (layer F.Cu) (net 41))
 (segment (start 145.36 124.6) (end 148.42 121.54) (width 0.1524) (layer F.Cu) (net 41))
 (segment (start 123.85 125.65) (end 124.9 124.6) (width 0.1524) (layer F.Cu) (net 41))
 (segment (start 147.5 125) (end 150.96 121.54) (width 0.1524) (layer F.Cu) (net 42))
 (segment (start 125.5 125) (end 147.5 125) (width 0.1524) (layer F.Cu) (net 42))
 (segment (start 124.65 127.1) (end 124.65 125.85) (width 0.1524) (layer F.Cu) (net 42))
 (segment (start 124.65 125.85) (end 125.5 125) (width 0.1524) (layer F.Cu) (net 42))
 (segment (start 149.7 116.685) (end 149.5 116.485) (width 0.1524) (layer F.Cu) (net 42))
 (segment (start 150.96 121.54) (end 149.7 120.28) (width 0.1524) (layer F.Cu) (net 42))
 (segment (start 149.7 120.28) (end 149.7 116.685) (width 0.1524) (layer F.Cu) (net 42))
 (segment (start 149.64 125.4) (end 153.5 121.54) (width 0.1524) (layer F.Cu) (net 43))
 (segment (start 126.1 125.4) (end 149.64 125.4) (width 0.1524) (layer F.Cu) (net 43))
 (segment (start 125.45 127.1) (end 125.45 126.05) (width 0.1524) (layer F.Cu) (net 43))
 (segment (start 125.45 126.05) (end 126.1 125.4) (width 0.1524) (layer F.Cu) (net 43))
 (segment (start 153.5 121.54) (end 152.2 120.24) (width 0.1524) (layer F.Cu) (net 43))
 (segment (start 152.2 116.685) (end 152 116.485) (width 0.1524) (layer F.Cu) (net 43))
 (segment (start 152.2 120.24) (end 152.2 116.685) (width 0.1524) (layer F.Cu) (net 43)))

